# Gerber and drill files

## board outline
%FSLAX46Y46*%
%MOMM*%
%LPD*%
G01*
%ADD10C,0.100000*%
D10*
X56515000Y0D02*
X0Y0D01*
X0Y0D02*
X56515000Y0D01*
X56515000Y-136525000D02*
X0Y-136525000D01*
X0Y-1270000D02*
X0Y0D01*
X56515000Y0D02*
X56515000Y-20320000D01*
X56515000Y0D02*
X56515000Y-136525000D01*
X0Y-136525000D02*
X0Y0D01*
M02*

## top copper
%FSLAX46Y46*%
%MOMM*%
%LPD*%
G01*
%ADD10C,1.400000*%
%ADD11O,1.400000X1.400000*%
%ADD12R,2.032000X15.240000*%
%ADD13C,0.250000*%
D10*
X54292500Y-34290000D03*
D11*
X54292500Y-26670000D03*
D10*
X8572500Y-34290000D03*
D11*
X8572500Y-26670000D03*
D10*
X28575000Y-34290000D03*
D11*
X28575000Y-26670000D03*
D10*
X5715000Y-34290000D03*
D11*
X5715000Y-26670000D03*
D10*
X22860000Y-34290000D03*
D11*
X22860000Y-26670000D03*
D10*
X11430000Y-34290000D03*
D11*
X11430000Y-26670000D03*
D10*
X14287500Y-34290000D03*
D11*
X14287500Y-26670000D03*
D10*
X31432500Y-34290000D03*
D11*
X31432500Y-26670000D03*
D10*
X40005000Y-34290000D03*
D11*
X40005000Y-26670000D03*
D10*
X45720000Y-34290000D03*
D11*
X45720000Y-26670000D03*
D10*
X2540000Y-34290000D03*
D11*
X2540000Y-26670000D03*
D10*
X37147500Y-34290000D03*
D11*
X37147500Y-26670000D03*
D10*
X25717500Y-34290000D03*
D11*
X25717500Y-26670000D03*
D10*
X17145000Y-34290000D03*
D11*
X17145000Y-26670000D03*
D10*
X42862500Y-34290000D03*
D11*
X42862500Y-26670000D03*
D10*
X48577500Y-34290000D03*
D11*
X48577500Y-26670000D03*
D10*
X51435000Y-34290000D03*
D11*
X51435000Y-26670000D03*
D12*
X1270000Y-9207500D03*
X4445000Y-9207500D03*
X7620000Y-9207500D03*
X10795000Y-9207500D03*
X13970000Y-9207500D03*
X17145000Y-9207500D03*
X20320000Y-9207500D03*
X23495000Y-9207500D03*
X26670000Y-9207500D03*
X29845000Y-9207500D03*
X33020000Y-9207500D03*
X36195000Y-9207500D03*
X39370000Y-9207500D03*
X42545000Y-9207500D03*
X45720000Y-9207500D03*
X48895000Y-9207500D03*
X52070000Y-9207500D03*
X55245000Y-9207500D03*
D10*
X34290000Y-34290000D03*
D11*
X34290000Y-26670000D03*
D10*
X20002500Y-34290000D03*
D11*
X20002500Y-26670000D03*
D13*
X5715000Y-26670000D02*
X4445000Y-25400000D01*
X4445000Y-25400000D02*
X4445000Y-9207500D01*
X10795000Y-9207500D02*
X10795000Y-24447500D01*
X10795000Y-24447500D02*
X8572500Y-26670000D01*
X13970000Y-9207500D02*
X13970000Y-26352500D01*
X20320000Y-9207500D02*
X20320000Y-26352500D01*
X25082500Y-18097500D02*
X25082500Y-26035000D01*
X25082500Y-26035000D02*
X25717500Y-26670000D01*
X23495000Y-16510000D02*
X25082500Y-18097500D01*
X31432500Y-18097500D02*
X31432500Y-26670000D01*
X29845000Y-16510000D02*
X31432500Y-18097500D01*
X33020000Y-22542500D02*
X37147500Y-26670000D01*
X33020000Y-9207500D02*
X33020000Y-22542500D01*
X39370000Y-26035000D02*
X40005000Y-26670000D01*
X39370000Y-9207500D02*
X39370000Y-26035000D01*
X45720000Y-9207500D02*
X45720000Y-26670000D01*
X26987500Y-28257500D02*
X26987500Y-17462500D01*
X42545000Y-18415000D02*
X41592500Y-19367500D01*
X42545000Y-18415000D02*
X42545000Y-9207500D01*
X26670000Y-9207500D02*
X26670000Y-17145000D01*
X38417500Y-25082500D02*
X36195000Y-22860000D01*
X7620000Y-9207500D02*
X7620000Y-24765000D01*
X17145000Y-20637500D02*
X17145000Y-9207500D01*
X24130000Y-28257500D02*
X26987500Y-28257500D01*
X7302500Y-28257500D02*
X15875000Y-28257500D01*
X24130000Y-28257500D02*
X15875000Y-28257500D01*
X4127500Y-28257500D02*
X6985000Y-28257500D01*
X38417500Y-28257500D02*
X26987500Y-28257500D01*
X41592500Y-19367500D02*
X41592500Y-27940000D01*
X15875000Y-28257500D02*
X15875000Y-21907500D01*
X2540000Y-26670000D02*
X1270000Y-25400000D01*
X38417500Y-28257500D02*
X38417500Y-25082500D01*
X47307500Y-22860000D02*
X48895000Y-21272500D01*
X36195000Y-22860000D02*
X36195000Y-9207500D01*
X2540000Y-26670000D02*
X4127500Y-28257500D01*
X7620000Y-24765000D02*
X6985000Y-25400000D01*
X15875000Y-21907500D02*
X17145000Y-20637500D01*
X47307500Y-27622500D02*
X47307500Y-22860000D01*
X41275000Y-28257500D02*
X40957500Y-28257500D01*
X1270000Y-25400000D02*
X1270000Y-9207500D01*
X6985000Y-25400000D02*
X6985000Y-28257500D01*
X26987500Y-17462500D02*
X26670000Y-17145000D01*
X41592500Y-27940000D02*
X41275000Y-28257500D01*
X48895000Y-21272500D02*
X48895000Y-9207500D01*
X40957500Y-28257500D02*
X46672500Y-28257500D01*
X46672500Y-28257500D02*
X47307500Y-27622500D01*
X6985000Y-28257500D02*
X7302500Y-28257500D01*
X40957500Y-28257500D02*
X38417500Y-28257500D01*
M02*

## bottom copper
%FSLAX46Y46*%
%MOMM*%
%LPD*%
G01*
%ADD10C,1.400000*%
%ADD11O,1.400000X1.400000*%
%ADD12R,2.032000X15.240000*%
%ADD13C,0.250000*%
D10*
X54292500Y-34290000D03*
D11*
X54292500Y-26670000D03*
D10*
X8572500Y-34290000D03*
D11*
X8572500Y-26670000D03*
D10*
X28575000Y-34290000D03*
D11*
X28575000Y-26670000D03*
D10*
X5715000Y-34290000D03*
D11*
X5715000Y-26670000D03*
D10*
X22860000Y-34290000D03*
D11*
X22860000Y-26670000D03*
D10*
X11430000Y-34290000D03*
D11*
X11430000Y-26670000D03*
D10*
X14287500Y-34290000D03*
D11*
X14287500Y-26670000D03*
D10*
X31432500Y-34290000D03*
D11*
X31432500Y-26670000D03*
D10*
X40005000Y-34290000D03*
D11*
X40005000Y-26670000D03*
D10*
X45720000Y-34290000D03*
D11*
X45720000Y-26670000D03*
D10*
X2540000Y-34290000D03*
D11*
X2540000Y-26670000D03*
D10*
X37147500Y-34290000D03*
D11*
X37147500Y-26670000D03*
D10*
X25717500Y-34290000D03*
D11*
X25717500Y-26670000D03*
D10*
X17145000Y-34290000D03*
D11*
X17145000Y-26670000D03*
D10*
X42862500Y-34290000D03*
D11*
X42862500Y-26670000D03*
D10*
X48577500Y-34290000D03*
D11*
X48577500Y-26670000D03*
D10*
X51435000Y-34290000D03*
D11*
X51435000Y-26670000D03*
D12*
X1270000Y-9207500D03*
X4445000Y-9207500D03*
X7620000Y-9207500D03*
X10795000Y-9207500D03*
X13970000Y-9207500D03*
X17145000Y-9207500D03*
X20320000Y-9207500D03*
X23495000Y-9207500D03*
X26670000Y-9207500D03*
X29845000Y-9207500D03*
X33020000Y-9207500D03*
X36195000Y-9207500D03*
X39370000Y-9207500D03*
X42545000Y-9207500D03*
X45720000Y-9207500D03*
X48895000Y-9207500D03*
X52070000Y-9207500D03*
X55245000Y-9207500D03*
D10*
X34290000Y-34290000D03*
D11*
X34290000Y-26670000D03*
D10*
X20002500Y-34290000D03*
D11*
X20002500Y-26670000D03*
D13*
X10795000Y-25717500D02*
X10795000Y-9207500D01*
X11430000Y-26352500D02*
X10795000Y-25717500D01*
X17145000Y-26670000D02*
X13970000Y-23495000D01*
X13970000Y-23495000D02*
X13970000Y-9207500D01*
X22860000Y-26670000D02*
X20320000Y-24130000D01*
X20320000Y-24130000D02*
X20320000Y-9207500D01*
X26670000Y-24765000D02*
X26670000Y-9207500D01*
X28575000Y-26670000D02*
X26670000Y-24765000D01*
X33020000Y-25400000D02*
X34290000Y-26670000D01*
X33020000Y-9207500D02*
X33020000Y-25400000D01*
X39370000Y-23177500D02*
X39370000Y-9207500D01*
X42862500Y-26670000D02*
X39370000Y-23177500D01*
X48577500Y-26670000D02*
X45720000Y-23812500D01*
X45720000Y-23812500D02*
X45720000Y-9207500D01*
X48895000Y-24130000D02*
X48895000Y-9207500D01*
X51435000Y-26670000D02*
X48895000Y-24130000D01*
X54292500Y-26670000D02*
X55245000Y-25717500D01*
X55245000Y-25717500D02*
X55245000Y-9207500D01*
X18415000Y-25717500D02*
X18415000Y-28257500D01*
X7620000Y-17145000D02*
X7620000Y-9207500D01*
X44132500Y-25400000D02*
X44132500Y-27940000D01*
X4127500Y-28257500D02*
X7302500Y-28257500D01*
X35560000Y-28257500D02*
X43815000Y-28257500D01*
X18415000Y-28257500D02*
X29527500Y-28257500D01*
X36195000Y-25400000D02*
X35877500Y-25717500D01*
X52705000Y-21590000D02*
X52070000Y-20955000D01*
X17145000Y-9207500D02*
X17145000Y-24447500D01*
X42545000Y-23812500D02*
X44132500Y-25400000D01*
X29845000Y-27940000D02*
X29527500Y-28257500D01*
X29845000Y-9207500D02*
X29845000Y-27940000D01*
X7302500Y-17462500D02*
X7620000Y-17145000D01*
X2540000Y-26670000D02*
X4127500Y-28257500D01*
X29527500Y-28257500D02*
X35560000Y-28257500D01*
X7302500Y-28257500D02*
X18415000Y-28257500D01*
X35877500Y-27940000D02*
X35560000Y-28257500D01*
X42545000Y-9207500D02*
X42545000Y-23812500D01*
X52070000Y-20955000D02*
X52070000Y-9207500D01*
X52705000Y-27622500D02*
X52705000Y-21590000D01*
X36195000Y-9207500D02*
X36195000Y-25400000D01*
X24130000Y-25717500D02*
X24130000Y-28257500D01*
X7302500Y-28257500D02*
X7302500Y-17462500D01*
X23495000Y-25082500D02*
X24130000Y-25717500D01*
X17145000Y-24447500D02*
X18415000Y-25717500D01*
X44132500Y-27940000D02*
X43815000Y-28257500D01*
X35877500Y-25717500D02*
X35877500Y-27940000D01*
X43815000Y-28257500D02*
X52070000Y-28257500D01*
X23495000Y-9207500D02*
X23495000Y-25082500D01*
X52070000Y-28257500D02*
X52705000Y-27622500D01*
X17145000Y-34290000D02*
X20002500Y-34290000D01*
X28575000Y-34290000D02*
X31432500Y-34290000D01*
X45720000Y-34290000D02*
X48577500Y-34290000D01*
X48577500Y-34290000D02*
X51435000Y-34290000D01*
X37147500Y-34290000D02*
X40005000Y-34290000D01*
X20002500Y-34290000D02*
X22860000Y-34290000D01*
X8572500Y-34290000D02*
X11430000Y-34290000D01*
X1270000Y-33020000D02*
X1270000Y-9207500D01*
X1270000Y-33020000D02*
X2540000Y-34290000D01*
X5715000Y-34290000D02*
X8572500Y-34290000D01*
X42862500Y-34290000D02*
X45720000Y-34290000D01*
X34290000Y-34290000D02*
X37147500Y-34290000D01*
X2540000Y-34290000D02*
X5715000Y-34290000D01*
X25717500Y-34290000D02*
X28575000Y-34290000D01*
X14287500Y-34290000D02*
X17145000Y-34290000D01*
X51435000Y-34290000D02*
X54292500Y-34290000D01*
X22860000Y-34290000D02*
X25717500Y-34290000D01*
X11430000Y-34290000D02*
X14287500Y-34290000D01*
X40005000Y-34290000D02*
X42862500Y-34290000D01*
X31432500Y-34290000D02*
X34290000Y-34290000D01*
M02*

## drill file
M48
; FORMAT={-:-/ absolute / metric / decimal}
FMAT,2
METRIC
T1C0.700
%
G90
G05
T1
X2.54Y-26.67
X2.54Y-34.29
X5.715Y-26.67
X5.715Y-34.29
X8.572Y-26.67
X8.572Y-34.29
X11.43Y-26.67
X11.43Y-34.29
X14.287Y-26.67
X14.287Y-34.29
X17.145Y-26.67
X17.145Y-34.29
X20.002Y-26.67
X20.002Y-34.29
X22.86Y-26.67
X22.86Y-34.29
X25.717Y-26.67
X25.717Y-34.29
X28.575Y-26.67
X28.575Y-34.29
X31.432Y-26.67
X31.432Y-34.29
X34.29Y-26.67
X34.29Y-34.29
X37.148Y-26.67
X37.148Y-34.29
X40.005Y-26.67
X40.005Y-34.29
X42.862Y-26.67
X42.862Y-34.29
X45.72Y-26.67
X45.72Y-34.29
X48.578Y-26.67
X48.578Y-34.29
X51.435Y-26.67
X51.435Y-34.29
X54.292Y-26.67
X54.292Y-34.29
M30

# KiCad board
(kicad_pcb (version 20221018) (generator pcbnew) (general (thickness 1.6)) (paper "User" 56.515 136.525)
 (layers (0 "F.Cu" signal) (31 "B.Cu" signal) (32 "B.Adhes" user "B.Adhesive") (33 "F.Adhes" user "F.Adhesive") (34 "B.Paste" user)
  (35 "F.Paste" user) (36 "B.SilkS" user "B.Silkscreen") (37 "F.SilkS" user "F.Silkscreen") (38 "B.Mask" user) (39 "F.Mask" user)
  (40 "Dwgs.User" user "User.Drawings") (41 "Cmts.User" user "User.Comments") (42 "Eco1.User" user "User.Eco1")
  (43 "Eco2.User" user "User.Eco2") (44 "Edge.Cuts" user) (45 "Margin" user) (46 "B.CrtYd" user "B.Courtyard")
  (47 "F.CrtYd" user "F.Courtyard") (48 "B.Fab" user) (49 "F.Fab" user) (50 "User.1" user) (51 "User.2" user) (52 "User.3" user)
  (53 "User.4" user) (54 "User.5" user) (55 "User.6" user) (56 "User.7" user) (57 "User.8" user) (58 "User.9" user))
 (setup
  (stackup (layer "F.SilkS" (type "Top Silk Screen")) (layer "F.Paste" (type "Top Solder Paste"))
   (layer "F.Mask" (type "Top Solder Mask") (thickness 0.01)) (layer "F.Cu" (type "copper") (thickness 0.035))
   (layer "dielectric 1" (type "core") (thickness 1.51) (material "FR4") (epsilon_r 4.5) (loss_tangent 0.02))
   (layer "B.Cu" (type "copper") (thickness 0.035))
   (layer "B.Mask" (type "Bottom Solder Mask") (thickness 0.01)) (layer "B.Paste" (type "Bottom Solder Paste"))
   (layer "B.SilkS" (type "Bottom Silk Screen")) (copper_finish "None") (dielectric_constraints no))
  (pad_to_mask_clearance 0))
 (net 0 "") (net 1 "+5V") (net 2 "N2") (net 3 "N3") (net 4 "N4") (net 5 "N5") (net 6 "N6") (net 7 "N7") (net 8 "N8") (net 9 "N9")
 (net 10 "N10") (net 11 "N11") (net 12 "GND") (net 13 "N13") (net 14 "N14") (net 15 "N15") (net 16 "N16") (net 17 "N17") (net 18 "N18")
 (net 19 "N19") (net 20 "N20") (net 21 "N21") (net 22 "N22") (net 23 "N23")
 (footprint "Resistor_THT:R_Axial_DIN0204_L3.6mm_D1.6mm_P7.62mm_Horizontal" (layer "F.Cu") (at 54.2925 34.29 90)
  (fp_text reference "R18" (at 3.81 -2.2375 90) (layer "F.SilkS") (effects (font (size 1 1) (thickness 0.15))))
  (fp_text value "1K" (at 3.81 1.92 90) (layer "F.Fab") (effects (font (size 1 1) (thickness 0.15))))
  (pad "1" thru_hole circle (at 0 0 90) (size 1.4 1.4) (drill 0.7) (layers "*.Cu" "*.Mask") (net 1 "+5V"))
  (pad "2" thru_hole oval (at 7.62 0 90) (size 1.4 1.4) (drill 0.7) (layers "*.Cu" "*.Mask") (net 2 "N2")))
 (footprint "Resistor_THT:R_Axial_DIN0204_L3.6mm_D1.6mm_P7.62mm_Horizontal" (layer "F.Cu") (at 8.5725 34.29 90)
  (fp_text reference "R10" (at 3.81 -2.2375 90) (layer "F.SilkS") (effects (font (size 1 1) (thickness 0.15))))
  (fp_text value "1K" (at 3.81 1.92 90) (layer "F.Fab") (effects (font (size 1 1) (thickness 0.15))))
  (pad "1" thru_hole circle (at 0 0 90) (size 1.4 1.4) (drill 0.7) (layers "*.Cu" "*.Mask") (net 1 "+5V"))
  (pad "2" thru_hole oval (at 7.62 0 90) (size 1.4 1.4) (drill 0.7) (layers "*.Cu" "*.Mask") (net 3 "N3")))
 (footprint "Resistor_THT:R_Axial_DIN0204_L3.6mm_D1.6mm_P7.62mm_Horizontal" (layer "F.Cu") (at 28.575 34.29 90)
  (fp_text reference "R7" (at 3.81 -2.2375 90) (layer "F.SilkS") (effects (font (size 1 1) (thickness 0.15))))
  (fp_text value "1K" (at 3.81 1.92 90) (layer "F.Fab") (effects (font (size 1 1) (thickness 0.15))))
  (pad "1" thru_hole circle (at 0 0 90) (size 1.4 1.4) (drill 0.7) (layers "*.Cu" "*.Mask") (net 1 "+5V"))
  (pad "2" thru_hole oval (at 7.62 0 90) (size 1.4 1.4) (drill 0.7) (layers "*.Cu" "*.Mask") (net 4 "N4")))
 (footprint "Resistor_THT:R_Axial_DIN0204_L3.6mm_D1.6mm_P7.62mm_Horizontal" (layer "F.Cu") (at 5.715 34.29 90)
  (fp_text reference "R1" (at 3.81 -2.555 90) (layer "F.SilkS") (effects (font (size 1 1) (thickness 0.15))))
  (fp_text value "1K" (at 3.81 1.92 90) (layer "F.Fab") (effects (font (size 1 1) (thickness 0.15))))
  (pad "1" thru_hole circle (at 0 0 90) (size 1.4 1.4) (drill 0.7) (layers "*.Cu" "*.Mask") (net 1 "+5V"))
  (pad "2" thru_hole oval (at 7.62 0 90) (size 1.4 1.4) (drill 0.7) (layers "*.Cu" "*.Mask") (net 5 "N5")))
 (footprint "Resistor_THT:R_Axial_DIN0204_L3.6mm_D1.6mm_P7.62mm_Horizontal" (layer "F.Cu") (at 22.86 34.29 90)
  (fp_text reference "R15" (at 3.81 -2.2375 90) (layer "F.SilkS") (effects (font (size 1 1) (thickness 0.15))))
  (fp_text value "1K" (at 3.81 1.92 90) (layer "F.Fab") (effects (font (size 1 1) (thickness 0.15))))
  (pad "1" thru_hole circle (at 0 0 90) (size 1.4 1.4) (drill 0.7) (layers "*.Cu" "*.Mask") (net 1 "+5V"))
  (pad "2" thru_hole oval (at 7.62 0 90) (size 1.4 1.4) (drill 0.7) (layers "*.Cu" "*.Mask") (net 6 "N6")))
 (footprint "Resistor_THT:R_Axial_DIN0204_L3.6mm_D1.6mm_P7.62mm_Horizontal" (layer "F.Cu") (at 11.43 34.29 90)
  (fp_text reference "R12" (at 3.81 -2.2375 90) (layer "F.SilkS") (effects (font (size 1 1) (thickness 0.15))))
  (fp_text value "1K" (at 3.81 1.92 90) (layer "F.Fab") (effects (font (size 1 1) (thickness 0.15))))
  (pad "1" thru_hole circle (at 0 0 90) (size 1.4 1.4) (drill 0.7) (layers "*.Cu" "*.Mask") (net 1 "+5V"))
  (pad "2" thru_hole oval (at 7.62 0 90) (size 1.4 1.4) (drill 0.7) (layers "*.Cu" "*.Mask") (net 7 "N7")))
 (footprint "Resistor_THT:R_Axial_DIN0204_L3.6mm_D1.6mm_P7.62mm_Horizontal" (layer "F.Cu") (at 14.2875 34.29 90)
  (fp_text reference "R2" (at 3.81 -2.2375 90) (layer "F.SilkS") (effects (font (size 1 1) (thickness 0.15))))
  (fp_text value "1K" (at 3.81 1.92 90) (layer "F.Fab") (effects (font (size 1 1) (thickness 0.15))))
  (pad "1" thru_hole circle (at 0 0 90) (size 1.4 1.4) (drill 0.7) (layers "*.Cu" "*.Mask") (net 1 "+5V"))
  (pad "2" thru_hole oval (at 7.62 0 90) (size 1.4 1.4) (drill 0.7) (layers "*.Cu" "*.Mask") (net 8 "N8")))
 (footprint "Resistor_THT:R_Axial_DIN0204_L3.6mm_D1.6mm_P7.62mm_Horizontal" (layer "F.Cu") (at 31.4325 34.29 90)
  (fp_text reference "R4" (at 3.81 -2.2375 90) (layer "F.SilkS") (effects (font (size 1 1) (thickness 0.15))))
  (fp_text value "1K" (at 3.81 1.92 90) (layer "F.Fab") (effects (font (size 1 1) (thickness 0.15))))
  (pad "1" thru_hole circle (at 0 0 90) (size 1.4 1.4) (drill 0.7) (layers "*.Cu" "*.Mask") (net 1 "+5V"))
  (pad "2" thru_hole oval (at 7.62 0 90) (size 1.4 1.4) (drill 0.7) (layers "*.Cu" "*.Mask") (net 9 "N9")))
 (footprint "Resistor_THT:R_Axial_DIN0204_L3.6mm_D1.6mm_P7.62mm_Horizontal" (layer "F.Cu") (at 40.005 34.29 90)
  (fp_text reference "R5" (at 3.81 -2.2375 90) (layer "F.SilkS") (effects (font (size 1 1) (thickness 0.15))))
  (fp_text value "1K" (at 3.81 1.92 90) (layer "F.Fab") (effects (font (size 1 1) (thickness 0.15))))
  (pad "1" thru_hole circle (at 0 0 90) (size 1.4 1.4) (drill 0.7) (layers "*.Cu" "*.Mask") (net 1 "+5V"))
  (pad "2" thru_hole oval (at 7.62 0 90) (size 1.4 1.4) (drill 0.7) (layers "*.Cu" "*.Mask") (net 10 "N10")))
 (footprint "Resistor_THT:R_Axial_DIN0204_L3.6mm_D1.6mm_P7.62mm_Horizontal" (layer "F.Cu") (at 45.72 34.29 90)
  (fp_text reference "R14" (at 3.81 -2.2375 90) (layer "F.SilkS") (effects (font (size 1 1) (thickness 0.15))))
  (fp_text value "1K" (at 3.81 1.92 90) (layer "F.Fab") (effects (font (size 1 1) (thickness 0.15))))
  (pad "1" thru_hole circle (at 0 0 90) (size 1.4 1.4) (drill 0.7) (layers "*.Cu" "*.Mask") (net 1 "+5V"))
  (pad "2" thru_hole oval (at 7.62 0 90) (size 1.4 1.4) (drill 0.7) (layers "*.Cu" "*.Mask") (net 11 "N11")))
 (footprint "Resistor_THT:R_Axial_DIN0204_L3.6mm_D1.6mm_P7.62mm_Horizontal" (layer "F.Cu") (at 2.54 34.29 90)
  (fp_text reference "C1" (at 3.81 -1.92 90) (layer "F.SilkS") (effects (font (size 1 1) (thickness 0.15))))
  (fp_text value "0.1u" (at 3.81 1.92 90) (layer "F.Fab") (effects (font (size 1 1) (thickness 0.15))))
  (pad "1" thru_hole circle (at 0 0 90) (size 1.4 1.4) (drill 0.7) (layers "*.Cu" "*.Mask") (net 1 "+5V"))
  (pad "2" thru_hole oval (at 7.62 0 90) (size 1.4 1.4) (drill 0.7) (layers "*.Cu" "*.Mask") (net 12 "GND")))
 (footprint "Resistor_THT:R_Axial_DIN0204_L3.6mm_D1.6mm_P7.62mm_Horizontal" (layer "F.Cu") (at 37.1475 34.29 90)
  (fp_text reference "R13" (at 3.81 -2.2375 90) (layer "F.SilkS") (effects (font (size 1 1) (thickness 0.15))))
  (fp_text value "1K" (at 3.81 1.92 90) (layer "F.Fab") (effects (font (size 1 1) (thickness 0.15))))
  (pad "1" thru_hole circle (at 0 0 90) (size 1.4 1.4) (drill 0.7) (layers "*.Cu" "*.Mask") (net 1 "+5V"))
  (pad "2" thru_hole oval (at 7.62 0 90) (size 1.4 1.4) (drill 0.7) (layers "*.Cu" "*.Mask") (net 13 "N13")))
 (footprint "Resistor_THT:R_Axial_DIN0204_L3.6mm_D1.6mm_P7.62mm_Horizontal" (layer "F.Cu") (at 25.7175 34.29 90)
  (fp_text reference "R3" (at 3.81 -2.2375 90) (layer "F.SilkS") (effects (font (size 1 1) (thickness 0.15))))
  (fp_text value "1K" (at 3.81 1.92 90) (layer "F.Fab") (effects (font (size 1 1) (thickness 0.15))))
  (pad "1" thru_hole circle (at 0 0 90) (size 1.4 1.4) (drill 0.7) (layers "*.Cu" "*.Mask") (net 1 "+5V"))
  (pad "2" thru_hole oval (at 7.62 0 90) (size 1.4 1.4) (drill 0.7) (layers "*.Cu" "*.Mask") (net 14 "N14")))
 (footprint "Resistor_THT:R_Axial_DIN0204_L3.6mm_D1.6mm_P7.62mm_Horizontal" (layer "F.Cu") (at 17.145 34.29 90)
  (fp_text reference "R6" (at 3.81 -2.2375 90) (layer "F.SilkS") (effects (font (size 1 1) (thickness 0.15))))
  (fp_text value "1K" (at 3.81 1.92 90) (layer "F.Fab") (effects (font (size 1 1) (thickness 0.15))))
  (pad "1" thru_hole circle (at 0 0 90) (size 1.4 1.4) (drill 0.7) (layers "*.Cu" "*.Mask") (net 1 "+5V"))
  (pad "2" thru_hole oval (at 7.62 0 90) (size 1.4 1.4) (drill 0.7) (layers "*.Cu" "*.Mask") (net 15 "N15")))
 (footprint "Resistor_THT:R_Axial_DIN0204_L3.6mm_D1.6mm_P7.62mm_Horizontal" (layer "F.Cu") (at 42.8625 34.29 90)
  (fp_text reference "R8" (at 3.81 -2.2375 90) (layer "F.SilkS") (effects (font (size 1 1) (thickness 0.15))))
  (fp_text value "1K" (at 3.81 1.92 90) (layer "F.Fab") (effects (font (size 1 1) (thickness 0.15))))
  (pad "1" thru_hole circle (at 0 0 90) (size 1.4 1.4) (drill 0.7) (layers "*.Cu" "*.Mask") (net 1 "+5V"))
  (pad "2" thru_hole oval (at 7.62 0 90) (size 1.4 1.4) (drill 0.7) (layers "*.Cu" "*.Mask") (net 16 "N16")))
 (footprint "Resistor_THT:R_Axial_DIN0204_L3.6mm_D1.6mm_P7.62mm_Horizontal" (layer "F.Cu") (at 48.5775 34.29 90)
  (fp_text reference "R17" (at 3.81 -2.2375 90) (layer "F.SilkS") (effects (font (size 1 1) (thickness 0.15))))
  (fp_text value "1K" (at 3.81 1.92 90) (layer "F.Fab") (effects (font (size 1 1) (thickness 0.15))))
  (pad "1" thru_hole circle (at 0 0 90) (size 1.4 1.4) (drill 0.7) (layers "*.Cu" "*.Mask") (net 1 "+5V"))
  (pad "2" thru_hole oval (at 7.62 0 90) (size 1.4 1.4) (drill 0.7) (layers "*.Cu" "*.Mask") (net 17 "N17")))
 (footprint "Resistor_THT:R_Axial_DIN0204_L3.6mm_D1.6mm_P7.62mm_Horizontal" (layer "F.Cu") (at 51.435 34.29 90)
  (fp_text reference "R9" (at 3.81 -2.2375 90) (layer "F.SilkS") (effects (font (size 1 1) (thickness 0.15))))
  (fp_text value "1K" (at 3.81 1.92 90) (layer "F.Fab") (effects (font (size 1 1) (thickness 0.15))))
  (pad "1" thru_hole circle (at 0 0 90) (size 1.4 1.4) (drill 0.7) (layers "*.Cu" "*.Mask") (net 1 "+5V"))
  (pad "2" thru_hole oval (at 7.62 0 90) (size 1.4 1.4) (drill 0.7) (layers "*.Cu" "*.Mask") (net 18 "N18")))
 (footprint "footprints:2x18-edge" (layer "F.Cu") (at 55.245 9.2075)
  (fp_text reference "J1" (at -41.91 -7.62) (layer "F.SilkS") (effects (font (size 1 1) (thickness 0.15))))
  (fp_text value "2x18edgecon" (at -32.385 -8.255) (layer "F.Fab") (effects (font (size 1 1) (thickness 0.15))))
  (pad "A1" connect rect (at -53.975 0) (size 2.032 15.24) (layers "F.Cu" "F.Mask") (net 12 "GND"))
  (pad "A2" connect rect (at -53.975 0) (size 2.032 15.24) (layers "B.Cu" "B.Mask") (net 1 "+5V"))
  (pad "B1" connect rect (at -50.8 0) (size 2.032 15.24) (layers "F.Cu" "F.Mask") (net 5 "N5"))
  (pad "B2" connect rect (at -50.8 0) (size 2.032 15.24) (layers "B.Cu" "B.Mask") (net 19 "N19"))
  (pad "C1" connect rect (at -47.625 0) (size 2.032 15.24) (layers "F.Cu" "F.Mask") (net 12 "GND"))
  (pad "C2" connect rect (at -47.625 0) (size 2.032 15.24) (layers "B.Cu" "B.Mask") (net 12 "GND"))
  (pad "D1" connect rect (at -44.45 0) (size 2.032 15.24) (layers "F.Cu" "F.Mask") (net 3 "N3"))
  (pad "D2" connect rect (at -44.45 0) (size 2.032 15.24) (layers "B.Cu" "B.Mask") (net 7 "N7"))
  (pad "E1" connect rect (at -41.275 0) (size 2.032 15.24) (layers "F.Cu" "F.Mask") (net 8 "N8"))
  (pad "E2" connect rect (at -41.275 0) (size 2.032 15.24) (layers "B.Cu" "B.Mask") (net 15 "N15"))
  (pad "F1" connect rect (at -38.1 0) (size 2.032 15.24) (layers "F.Cu" "F.Mask") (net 12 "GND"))
  (pad "F2" connect rect (at -38.1 0) (size 2.032 15.24) (layers "B.Cu" "B.Mask") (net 12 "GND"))
  (pad "H1" connect rect (at -34.925 0) (size 2.032 15.24) (layers "F.Cu" "F.Mask") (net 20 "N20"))
  (pad "H2" connect rect (at -34.925 0) (size 2.032 15.24) (layers "B.Cu" "B.Mask") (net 6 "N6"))
  (pad "J1" connect rect (at -31.75 0) (size 2.032 15.24) (layers "F.Cu" "F.Mask") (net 14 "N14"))
  (pad "J2" connect rect (at -31.75 0) (size 2.032 15.24) (layers "B.Cu" "B.Mask") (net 12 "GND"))
  (pad "K1" connect rect (at -28.575 0) (size 2.032 15.24) (layers "F.Cu" "F.Mask") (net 12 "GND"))
  (pad "K2" connect rect (at -28.575 0) (size 2.032 15.24) (layers "B.Cu" "B.Mask") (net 4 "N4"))
  (pad "L1" connect rect (at -25.4 0) (size 2.032 15.24) (layers "F.Cu" "F.Mask") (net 9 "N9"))
  (pad "L2" connect rect (at -25.4 0) (size 2.032 15.24) (layers "B.Cu" "B.Mask") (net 12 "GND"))
  (pad "M1" connect rect (at -22.225 0) (size 2.032 15.24) (layers "F.Cu" "F.Mask") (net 13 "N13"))
  (pad "M2" connect rect (at -22.225 0) (size 2.032 15.24) (layers "B.Cu" "B.Mask") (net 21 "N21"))
  (pad "N1" connect rect (at -19.05 0) (size 2.032 15.24) (layers "F.Cu" "F.Mask") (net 12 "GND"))
  (pad "N2" connect rect (at -19.05 0) (size 2.032 15.24) (layers "B.Cu" "B.Mask") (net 12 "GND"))
  (pad "P1" connect rect (at -15.875 0) (size 2.032 15.24) (layers "F.Cu" "F.Mask") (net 10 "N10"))
  (pad "P2" connect rect (at -15.875 0) (size 2.032 15.24) (layers "B.Cu" "B.Mask") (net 16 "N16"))
  (pad "R1" connect rect (at -12.7 0) (size 2.032 15.24) (layers "F.Cu" "F.Mask") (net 12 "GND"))
  (pad "R2" connect rect (at -12.7 0) (size 2.032 15.24) (layers "B.Cu" "B.Mask") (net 12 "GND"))
  (pad "S1" connect rect (at -9.525 0) (size 2.032 15.24) (layers "F.Cu" "F.Mask") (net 11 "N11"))
  (pad "S2" connect rect (at -9.525 0) (size 2.032 15.24) (layers "B.Cu" "B.Mask") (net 17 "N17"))
  (pad "T1" connect rect (at -6.35 0) (size 2.032 15.24) (layers "F.Cu" "F.Mask") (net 12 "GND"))
  (pad "T2" connect rect (at -6.35 0) (size 2.032 15.24) (layers "B.Cu" "B.Mask") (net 18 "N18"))
  (pad "U1" connect rect (at -3.175 0) (size 2.032 15.24) (layers "F.Cu" "F.Mask") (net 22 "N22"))
  (pad "U2" connect rect (at -3.175 0) (size 2.032 15.24) (layers "B.Cu" "B.Mask") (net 12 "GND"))
  (pad "V1" connect rect (at 0 0) (size 2.032 15.24) (layers "F.Cu" "F.Mask") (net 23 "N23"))
  (pad "V2" connect rect (at 0 0) (size 2.032 15.24) (layers "B.Cu" "B.Mask") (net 2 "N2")))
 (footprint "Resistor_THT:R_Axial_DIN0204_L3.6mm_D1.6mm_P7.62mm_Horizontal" (layer "F.Cu") (at 34.29 34.29 90)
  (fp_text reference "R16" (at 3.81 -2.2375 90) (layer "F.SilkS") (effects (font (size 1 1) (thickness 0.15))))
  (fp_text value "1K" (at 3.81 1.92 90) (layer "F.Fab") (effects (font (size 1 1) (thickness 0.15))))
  (pad "1" thru_hole circle (at 0 0 90) (size 1.4 1.4) (drill 0.7) (layers "*.Cu" "*.Mask") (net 1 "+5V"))
  (pad "2" thru_hole oval (at 7.62 0 90) (size 1.4 1.4) (drill 0.7) (layers "*.Cu" "*.Mask") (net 21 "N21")))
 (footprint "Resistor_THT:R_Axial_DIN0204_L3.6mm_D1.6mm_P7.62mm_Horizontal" (layer "F.Cu") (at 20.0025 34.29 90)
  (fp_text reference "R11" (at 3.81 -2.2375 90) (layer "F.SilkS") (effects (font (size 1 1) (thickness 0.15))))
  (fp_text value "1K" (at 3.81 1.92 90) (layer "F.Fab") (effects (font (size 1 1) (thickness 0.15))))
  (pad "1" thru_hole circle (at 0 0 90) (size 1.4 1.4) (drill 0.7) (layers "*.Cu" "*.Mask") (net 1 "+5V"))
  (pad "2" thru_hole oval (at 7.62 0 90) (size 1.4 1.4) (drill 0.7) (layers "*.Cu" "*.Mask") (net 20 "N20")))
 (gr_line (start 56.515 0) (end 0 0) (stroke (width 0.1) (type default)) (layer "Edge.Cuts"))
 (gr_line (start 0 0) (end 56.515 0) (stroke (width 0.1) (type default)) (layer "Edge.Cuts"))
 (gr_line (start 56.515 136.525) (end 0 136.525) (stroke (width 0.1) (type default)) (layer "Edge.Cuts"))
 (gr_line (start 0 1.27) (end 0 0) (stroke (width 0.1) (type default)) (layer "Edge.Cuts"))
 (gr_line (start 56.515 0) (end 56.515 20.32) (stroke (width 0.1) (type default)) (layer "Edge.Cuts"))
 (gr_line (start 56.515 0) (end 56.515 136.525) (stroke (width 0.1) (type default)) (layer "Edge.Cuts"))
 (gr_line (start 0 136.525) (end 0 0) (stroke (width 0.1) (type default)) (layer "Edge.Cuts"))
 (segment (start 5.715 26.67) (end 4.445 25.4) (width 0.25) (layer "F.Cu") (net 5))
 (segment (start 4.445 25.4) (end 4.445 9.2075) (width 0.25) (layer "F.Cu") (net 5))
 (segment (start 10.795 9.2075) (end 10.795 24.4475) (width 0.25) (layer "F.Cu") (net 3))
 (segment (start 10.795 24.4475) (end 8.5725 26.67) (width 0.25) (layer "F.Cu") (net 3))
 (segment (start 10.795 25.7175) (end 10.795 9.2075) (width 0.25) (layer "B.Cu") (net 7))
 (segment (start 11.43 26.3525) (end 10.795 25.7175) (width 0.25) (layer "B.Cu") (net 7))
 (segment (start 13.97 9.2075) (end 13.97 26.3525) (width 0.25) (layer "F.Cu") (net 8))
 (segment (start 17.145 26.67) (end 13.97 23.495) (width 0.25) (layer "B.Cu") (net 15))
 (segment (start 13.97 23.495) (end 13.97 9.2075) (width 0.25) (layer "B.Cu") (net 15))
 (segment (start 20.32 9.2075) (end 20.32 26.3525) (width 0.25) (layer "F.Cu") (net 20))
 (segment (start 22.86 26.67) (end 20.32 24.13) (width 0.25) (layer "B.Cu") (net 6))
 (segment (start 20.32 24.13) (end 20.32 9.2075) (width 0.25) (layer "B.Cu") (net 6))
 (segment (start 25.0825 18.0975) (end 25.0825 26.035) (width 0.25) (layer "F.Cu") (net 14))
 (segment (start 25.0825 26.035) (end 25.7175 26.67) (width 0.25) (layer "F.Cu") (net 14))
 (segment (start 23.495 16.51) (end 25.0825 18.0975) (width 0.25) (layer "F.Cu") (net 14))
 (segment (start 26.67 24.765) (end 26.67 9.2075) (width 0.25) (layer "B.Cu") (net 4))
 (segment (start 28.575 26.67) (end 26.67 24.765) (width 0.25) (layer "B.Cu") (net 4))
 (segment (start 31.4325 18.0975) (end 31.4325 26.67) (width 0.25) (layer "F.Cu") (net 9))
 (segment (start 29.845 16.51) (end 31.4325 18.0975) (width 0.25) (layer "F.Cu") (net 9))
 (segment (start 33.02 22.5425) (end 37.1475 26.67) (width 0.25) (layer "F.Cu") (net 13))
 (segment (start 33.02 9.2075) (end 33.02 22.5425) (width 0.25) (layer "F.Cu") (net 13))
 (segment (start 33.02 25.4) (end 34.29 26.67) (width 0.25) (layer "B.Cu") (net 21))
 (segment (start 33.02 9.2075) (end 33.02 25.4) (width 0.25) (layer "B.Cu") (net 21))
 (segment (start 39.37 26.035) (end 40.005 26.67) (width 0.25) (layer "F.Cu") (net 10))
 (segment (start 39.37 9.2075) (end 39.37 26.035) (width 0.25) (layer "F.Cu") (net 10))
 (segment (start 39.37 23.1775) (end 39.37 9.2075) (width 0.25) (layer "B.Cu") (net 16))
 (segment (start 42.8625 26.67) (end 39.37 23.1775) (width 0.25) (layer "B.Cu") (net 16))
 (segment (start 45.72 9.2075) (end 45.72 26.67) (width 0.25) (layer "F.Cu") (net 11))
 (segment (start 48.5775 26.67) (end 45.72 23.8125) (width 0.25) (layer "B.Cu") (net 17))
 (segment (start 45.72 23.8125) (end 45.72 9.2075) (width 0.25) (layer "B.Cu") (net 17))
 (segment (start 48.895 24.13) (end 48.895 9.2075) (width 0.25) (layer "B.Cu") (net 18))
 (segment (start 51.435 26.67) (end 48.895 24.13) (width 0.25) (layer "B.Cu") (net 18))
 (segment (start 54.2925 26.67) (end 55.245 25.7175) (width 0.25) (layer "B.Cu") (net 2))
 (segment (start 55.245 25.7175) (end 55.245 9.2075) (width 0.25) (layer "B.Cu") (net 2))
 (segment (start 26.9875 28.2575) (end 26.9875 17.4625) (width 0.25) (layer "F.Cu") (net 12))
 (segment (start 42.545 18.415) (end 41.5925 19.3675) (width 0.25) (layer "F.Cu") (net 12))
 (segment (start 42.545 18.415) (end 42.545 9.2075) (width 0.25) (layer "F.Cu") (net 12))
 (segment (start 26.67 9.2075) (end 26.67 17.145) (width 0.25) (layer "F.Cu") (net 12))
 (segment (start 38.4175 25.0825) (end 36.195 22.86) (width 0.25) (layer "F.Cu") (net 12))
 (segment (start 7.62 9.2075) (end 7.62 24.765) (width 0.25) (layer "F.Cu") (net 12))
 (segment (start 17.145 20.6375) (end 17.145 9.2075) (width 0.25) (layer "F.Cu") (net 12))
 (segment (start 24.13 28.2575) (end 26.9875 28.2575) (width 0.25) (layer "F.Cu") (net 12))
 (segment (start 7.3025 28.2575) (end 15.875 28.2575) (width 0.25) (layer "F.Cu") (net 12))
 (segment (start 24.13 28.2575) (end 15.875 28.2575) (width 0.25) (layer "F.Cu") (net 12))
 (segment (start 4.1275 28.2575) (end 6.985 28.2575) (width 0.25) (layer "F.Cu") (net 12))
 (segment (start 38.4175 28.2575) (end 26.9875 28.2575) (width 0.25) (layer "F.Cu") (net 12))
 (segment (start 41.5925 19.3675) (end 41.5925 27.94) (width 0.25) (layer "F.Cu") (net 12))
 (segment (start 15.875 28.2575) (end 15.875 21.9075) (width 0.25) (layer "F.Cu") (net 12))
 (segment (start 2.54 26.67) (end 1.27 25.4) (width 0.25) (layer "F.Cu") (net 12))
 (segment (start 38.4175 28.2575) (end 38.4175 25.0825) (width 0.25) (layer "F.Cu") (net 12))
 (segment (start 47.3075 22.86) (end 48.895 21.2725) (width 0.25) (layer "F.Cu") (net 12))
 (segment (start 36.195 22.86) (end 36.195 9.2075) (width 0.25) (layer "F.Cu") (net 12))
 (segment (start 2.54 26.67) (end 4.1275 28.2575) (width 0.25) (layer "F.Cu") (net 12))
 (segment (start 7.62 24.765) (end 6.985 25.4) (width 0.25) (layer "F.Cu") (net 12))
 (segment (start 15.875 21.9075) (end 17.145 20.6375) (width 0.25) (layer "F.Cu") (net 12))
 (segment (start 47.3075 27.6225) (end 47.3075 22.86) (width 0.25) (layer "F.Cu") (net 12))
 (segment (start 41.275 28.2575) (end 40.9575 28.2575) (width 0.25) (layer "F.Cu") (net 12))
 (segment (start 1.27 25.4) (end 1.27 9.2075) (width 0.25) (layer "F.Cu") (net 12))
 (segment (start 6.985 25.4) (end 6.985 28.2575) (width 0.25) (layer "F.Cu") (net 12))
 (segment (start 26.9875 17.4625) (end 26.67 17.145) (width 0.25) (layer "F.Cu") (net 12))
 (segment (start 41.5925 27.94) (end 41.275 28.2575) (width 0.25) (layer "F.Cu") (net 12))
 (segment (start 48.895 21.2725) (end 48.895 9.2075) (width 0.25) (layer "F.Cu") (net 12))
 (segment (start 40.9575 28.2575) (end 46.6725 28.2575) (width 0.25) (layer "F.Cu") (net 12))
 (segment (start 46.6725 28.2575) (end 47.3075 27.6225) (width 0.25) (layer "F.Cu") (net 12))
 (segment (start 6.985 28.2575) (end 7.3025 28.2575) (width 0.25) (layer "F.Cu") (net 12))
 (segment (start 40.9575 28.2575) (end 38.4175 28.2575) (width 0.25) (layer "F.Cu") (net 12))
 (segment (start 18.415 25.7175) (end 18.415 28.2575) (width 0.25) (layer "B.Cu") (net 12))
 (segment (start 7.62 17.145) (end 7.62 9.2075) (width 0.25) (layer "B.Cu") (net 12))
 (segment (start 44.1325 25.4) (end 44.1325 27.94) (width 0.25) (layer "B.Cu") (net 12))
 (segment (start 4.1275 28.2575) (end 7.3025 28.2575) (width 0.25) (layer "B.Cu") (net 12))
 (segment (start 35.56 28.2575) (end 43.815 28.2575) (width 0.25) (layer "B.Cu") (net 12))
 (segment (start 18.415 28.2575) (end 29.5275 28.2575) (width 0.25) (layer "B.Cu") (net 12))
 (segment (start 36.195 25.4) (end 35.8775 25.7175) (width 0.25) (layer "B.Cu") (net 12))
 (segment (start 52.705 21.59) (end 52.07 20.955) (width 0.25) (layer "B.Cu") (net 12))
 (segment (start 17.145 9.2075) (end 17.145 24.4475) (width 0.25) (layer "B.Cu") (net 12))
 (segment (start 42.545 23.8125) (end 44.1325 25.4) (width 0.25) (layer "B.Cu") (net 12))
 (segment (start 29.845 27.94) (end 29.5275 28.2575) (width 0.25) (layer "B.Cu") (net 12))
 (segment (start 29.845 9.2075) (end 29.845 27.94) (width 0.25) (layer "B.Cu") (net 12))
 (segment (start 7.3025 17.4625) (end 7.62 17.145) (width 0.25) (layer "B.Cu") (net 12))
 (segment (start 2.54 26.67) (end 4.1275 28.2575) (width 0.25) (layer "B.Cu") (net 12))
 (segment (start 29.5275 28.2575) (end 35.56 28.2575) (width 0.25) (layer "B.Cu") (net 12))
 (segment (start 7.3025 28.2575) (end 18.415 28.2575) (width 0.25) (layer "B.Cu") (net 12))
 (segment (start 35.8775 27.94) (end 35.56 28.2575) (width 0.25) (layer "B.Cu") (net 12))
 (segment (start 42.545 9.2075) (end 42.545 23.8125) (width 0.25) (layer "B.Cu") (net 12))
 (segment (start 52.07 20.955) (end 52.07 9.2075) (width 0.25) (layer "B.Cu") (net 12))
 (segment (start 52.705 27.6225) (end 52.705 21.59) (width 0.25) (layer "B.Cu") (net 12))
 (segment (start 36.195 9.2075) (end 36.195 25.4) (width 0.25) (layer "B.Cu") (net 12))
 (segment (start 24.13 25.7175) (end 24.13 28.2575) (width 0.25) (layer "B.Cu") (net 12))
 (segment (start 7.3025 28.2575) (end 7.3025 17.4625) (width 0.25) (layer "B.Cu") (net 12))
 (segment (start 23.495 25.0825) (end 24.13 25.7175) (width 0.25) (layer "B.Cu") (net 12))
 (segment (start 17.145 24.4475) (end 18.415 25.7175) (width 0.25) (layer "B.Cu") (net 12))
 (segment (start 44.1325 27.94) (end 43.815 28.2575) (width 0.25) (layer "B.Cu") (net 12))
 (segment (start 35.8775 25.7175) (end 35.8775 27.94) (width 0.25) (layer "B.Cu") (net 12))
 (segment (start 43.815 28.2575) (end 52.07 28.2575) (width 0.25) (layer "B.Cu") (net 12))
 (segment (start 23.495 9.2075) (end 23.495 25.0825) (width 0.25) (layer "B.Cu") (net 12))
 (segment (start 52.07 28.2575) (end 52.705 27.6225) (width 0.25) (layer "B.Cu") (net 12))
 (segment (start 17.145 34.29) (end 20.0025 34.29) (width 0.25) (layer "B.Cu") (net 1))
 (segment (start 28.575 34.29) (end 31.4325 34.29) (width 0.25) (layer "B.Cu") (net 1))
 (segment (start 45.72 34.29) (end 48.5775 34.29) (width 0.25) (layer "B.Cu") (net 1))
 (segment (start 48.5775 34.29) (end 51.435 34.29) (width 0.25) (layer "B.Cu") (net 1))
 (segment (start 37.1475 34.29) (end 40.005 34.29) (width 0.25) (layer "B.Cu") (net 1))
 (segment (start 20.0025 34.29) (end 22.86 34.29) (width 0.25) (layer "B.Cu") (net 1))
 (segment (start 8.5725 34.29) (end 11.43 34.29) (width 0.25) (layer "B.Cu") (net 1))
 (segment (start 1.27 33.02) (end 1.27 9.2075) (width 0.25) (layer "B.Cu") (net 1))
 (segment (start 1.27 33.02) (end 2.54 34.29) (width 0.25) (layer "B.Cu") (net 1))
 (segment (start 5.715 34.29) (end 8.5725 34.29) (width 0.25) (layer "B.Cu") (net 1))
 (segment (start 42.8625 34.29) (end 45.72 34.29) (width 0.25) (layer "B.Cu") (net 1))
 (segment (start 34.29 34.29) (end 37.1475 34.29) (width 0.25) (layer "B.Cu") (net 1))
 (segment (start 2.54 34.29) (end 5.715 34.29) (width 0.25) (layer "B.Cu") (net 1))
 (segment (start 25.7175 34.29) (end 28.575 34.29) (width 0.25) (layer "B.Cu") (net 1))
 (segment (start 14.2875 34.29) (end 17.145 34.29) (width 0.25) (layer "B.Cu") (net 1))
 (segment (start 51.435 34.29) (end 54.2925 34.29) (width 0.25) (layer "B.Cu") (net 1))
 (segment (start 22.86 34.29) (end 25.7175 34.29) (width 0.25) (layer "B.Cu") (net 1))
 (segment (start 11.43 34.29) (end 14.2875 34.29) (width 0.25) (layer "B.Cu") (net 1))
 (segment (start 40.005 34.29) (end 42.8625 34.29) (width 0.25) (layer "B.Cu") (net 1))
 (segment (start 31.4325 34.29) (end 34.29 34.29) (width 0.25) (layer "B.Cu") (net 1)))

